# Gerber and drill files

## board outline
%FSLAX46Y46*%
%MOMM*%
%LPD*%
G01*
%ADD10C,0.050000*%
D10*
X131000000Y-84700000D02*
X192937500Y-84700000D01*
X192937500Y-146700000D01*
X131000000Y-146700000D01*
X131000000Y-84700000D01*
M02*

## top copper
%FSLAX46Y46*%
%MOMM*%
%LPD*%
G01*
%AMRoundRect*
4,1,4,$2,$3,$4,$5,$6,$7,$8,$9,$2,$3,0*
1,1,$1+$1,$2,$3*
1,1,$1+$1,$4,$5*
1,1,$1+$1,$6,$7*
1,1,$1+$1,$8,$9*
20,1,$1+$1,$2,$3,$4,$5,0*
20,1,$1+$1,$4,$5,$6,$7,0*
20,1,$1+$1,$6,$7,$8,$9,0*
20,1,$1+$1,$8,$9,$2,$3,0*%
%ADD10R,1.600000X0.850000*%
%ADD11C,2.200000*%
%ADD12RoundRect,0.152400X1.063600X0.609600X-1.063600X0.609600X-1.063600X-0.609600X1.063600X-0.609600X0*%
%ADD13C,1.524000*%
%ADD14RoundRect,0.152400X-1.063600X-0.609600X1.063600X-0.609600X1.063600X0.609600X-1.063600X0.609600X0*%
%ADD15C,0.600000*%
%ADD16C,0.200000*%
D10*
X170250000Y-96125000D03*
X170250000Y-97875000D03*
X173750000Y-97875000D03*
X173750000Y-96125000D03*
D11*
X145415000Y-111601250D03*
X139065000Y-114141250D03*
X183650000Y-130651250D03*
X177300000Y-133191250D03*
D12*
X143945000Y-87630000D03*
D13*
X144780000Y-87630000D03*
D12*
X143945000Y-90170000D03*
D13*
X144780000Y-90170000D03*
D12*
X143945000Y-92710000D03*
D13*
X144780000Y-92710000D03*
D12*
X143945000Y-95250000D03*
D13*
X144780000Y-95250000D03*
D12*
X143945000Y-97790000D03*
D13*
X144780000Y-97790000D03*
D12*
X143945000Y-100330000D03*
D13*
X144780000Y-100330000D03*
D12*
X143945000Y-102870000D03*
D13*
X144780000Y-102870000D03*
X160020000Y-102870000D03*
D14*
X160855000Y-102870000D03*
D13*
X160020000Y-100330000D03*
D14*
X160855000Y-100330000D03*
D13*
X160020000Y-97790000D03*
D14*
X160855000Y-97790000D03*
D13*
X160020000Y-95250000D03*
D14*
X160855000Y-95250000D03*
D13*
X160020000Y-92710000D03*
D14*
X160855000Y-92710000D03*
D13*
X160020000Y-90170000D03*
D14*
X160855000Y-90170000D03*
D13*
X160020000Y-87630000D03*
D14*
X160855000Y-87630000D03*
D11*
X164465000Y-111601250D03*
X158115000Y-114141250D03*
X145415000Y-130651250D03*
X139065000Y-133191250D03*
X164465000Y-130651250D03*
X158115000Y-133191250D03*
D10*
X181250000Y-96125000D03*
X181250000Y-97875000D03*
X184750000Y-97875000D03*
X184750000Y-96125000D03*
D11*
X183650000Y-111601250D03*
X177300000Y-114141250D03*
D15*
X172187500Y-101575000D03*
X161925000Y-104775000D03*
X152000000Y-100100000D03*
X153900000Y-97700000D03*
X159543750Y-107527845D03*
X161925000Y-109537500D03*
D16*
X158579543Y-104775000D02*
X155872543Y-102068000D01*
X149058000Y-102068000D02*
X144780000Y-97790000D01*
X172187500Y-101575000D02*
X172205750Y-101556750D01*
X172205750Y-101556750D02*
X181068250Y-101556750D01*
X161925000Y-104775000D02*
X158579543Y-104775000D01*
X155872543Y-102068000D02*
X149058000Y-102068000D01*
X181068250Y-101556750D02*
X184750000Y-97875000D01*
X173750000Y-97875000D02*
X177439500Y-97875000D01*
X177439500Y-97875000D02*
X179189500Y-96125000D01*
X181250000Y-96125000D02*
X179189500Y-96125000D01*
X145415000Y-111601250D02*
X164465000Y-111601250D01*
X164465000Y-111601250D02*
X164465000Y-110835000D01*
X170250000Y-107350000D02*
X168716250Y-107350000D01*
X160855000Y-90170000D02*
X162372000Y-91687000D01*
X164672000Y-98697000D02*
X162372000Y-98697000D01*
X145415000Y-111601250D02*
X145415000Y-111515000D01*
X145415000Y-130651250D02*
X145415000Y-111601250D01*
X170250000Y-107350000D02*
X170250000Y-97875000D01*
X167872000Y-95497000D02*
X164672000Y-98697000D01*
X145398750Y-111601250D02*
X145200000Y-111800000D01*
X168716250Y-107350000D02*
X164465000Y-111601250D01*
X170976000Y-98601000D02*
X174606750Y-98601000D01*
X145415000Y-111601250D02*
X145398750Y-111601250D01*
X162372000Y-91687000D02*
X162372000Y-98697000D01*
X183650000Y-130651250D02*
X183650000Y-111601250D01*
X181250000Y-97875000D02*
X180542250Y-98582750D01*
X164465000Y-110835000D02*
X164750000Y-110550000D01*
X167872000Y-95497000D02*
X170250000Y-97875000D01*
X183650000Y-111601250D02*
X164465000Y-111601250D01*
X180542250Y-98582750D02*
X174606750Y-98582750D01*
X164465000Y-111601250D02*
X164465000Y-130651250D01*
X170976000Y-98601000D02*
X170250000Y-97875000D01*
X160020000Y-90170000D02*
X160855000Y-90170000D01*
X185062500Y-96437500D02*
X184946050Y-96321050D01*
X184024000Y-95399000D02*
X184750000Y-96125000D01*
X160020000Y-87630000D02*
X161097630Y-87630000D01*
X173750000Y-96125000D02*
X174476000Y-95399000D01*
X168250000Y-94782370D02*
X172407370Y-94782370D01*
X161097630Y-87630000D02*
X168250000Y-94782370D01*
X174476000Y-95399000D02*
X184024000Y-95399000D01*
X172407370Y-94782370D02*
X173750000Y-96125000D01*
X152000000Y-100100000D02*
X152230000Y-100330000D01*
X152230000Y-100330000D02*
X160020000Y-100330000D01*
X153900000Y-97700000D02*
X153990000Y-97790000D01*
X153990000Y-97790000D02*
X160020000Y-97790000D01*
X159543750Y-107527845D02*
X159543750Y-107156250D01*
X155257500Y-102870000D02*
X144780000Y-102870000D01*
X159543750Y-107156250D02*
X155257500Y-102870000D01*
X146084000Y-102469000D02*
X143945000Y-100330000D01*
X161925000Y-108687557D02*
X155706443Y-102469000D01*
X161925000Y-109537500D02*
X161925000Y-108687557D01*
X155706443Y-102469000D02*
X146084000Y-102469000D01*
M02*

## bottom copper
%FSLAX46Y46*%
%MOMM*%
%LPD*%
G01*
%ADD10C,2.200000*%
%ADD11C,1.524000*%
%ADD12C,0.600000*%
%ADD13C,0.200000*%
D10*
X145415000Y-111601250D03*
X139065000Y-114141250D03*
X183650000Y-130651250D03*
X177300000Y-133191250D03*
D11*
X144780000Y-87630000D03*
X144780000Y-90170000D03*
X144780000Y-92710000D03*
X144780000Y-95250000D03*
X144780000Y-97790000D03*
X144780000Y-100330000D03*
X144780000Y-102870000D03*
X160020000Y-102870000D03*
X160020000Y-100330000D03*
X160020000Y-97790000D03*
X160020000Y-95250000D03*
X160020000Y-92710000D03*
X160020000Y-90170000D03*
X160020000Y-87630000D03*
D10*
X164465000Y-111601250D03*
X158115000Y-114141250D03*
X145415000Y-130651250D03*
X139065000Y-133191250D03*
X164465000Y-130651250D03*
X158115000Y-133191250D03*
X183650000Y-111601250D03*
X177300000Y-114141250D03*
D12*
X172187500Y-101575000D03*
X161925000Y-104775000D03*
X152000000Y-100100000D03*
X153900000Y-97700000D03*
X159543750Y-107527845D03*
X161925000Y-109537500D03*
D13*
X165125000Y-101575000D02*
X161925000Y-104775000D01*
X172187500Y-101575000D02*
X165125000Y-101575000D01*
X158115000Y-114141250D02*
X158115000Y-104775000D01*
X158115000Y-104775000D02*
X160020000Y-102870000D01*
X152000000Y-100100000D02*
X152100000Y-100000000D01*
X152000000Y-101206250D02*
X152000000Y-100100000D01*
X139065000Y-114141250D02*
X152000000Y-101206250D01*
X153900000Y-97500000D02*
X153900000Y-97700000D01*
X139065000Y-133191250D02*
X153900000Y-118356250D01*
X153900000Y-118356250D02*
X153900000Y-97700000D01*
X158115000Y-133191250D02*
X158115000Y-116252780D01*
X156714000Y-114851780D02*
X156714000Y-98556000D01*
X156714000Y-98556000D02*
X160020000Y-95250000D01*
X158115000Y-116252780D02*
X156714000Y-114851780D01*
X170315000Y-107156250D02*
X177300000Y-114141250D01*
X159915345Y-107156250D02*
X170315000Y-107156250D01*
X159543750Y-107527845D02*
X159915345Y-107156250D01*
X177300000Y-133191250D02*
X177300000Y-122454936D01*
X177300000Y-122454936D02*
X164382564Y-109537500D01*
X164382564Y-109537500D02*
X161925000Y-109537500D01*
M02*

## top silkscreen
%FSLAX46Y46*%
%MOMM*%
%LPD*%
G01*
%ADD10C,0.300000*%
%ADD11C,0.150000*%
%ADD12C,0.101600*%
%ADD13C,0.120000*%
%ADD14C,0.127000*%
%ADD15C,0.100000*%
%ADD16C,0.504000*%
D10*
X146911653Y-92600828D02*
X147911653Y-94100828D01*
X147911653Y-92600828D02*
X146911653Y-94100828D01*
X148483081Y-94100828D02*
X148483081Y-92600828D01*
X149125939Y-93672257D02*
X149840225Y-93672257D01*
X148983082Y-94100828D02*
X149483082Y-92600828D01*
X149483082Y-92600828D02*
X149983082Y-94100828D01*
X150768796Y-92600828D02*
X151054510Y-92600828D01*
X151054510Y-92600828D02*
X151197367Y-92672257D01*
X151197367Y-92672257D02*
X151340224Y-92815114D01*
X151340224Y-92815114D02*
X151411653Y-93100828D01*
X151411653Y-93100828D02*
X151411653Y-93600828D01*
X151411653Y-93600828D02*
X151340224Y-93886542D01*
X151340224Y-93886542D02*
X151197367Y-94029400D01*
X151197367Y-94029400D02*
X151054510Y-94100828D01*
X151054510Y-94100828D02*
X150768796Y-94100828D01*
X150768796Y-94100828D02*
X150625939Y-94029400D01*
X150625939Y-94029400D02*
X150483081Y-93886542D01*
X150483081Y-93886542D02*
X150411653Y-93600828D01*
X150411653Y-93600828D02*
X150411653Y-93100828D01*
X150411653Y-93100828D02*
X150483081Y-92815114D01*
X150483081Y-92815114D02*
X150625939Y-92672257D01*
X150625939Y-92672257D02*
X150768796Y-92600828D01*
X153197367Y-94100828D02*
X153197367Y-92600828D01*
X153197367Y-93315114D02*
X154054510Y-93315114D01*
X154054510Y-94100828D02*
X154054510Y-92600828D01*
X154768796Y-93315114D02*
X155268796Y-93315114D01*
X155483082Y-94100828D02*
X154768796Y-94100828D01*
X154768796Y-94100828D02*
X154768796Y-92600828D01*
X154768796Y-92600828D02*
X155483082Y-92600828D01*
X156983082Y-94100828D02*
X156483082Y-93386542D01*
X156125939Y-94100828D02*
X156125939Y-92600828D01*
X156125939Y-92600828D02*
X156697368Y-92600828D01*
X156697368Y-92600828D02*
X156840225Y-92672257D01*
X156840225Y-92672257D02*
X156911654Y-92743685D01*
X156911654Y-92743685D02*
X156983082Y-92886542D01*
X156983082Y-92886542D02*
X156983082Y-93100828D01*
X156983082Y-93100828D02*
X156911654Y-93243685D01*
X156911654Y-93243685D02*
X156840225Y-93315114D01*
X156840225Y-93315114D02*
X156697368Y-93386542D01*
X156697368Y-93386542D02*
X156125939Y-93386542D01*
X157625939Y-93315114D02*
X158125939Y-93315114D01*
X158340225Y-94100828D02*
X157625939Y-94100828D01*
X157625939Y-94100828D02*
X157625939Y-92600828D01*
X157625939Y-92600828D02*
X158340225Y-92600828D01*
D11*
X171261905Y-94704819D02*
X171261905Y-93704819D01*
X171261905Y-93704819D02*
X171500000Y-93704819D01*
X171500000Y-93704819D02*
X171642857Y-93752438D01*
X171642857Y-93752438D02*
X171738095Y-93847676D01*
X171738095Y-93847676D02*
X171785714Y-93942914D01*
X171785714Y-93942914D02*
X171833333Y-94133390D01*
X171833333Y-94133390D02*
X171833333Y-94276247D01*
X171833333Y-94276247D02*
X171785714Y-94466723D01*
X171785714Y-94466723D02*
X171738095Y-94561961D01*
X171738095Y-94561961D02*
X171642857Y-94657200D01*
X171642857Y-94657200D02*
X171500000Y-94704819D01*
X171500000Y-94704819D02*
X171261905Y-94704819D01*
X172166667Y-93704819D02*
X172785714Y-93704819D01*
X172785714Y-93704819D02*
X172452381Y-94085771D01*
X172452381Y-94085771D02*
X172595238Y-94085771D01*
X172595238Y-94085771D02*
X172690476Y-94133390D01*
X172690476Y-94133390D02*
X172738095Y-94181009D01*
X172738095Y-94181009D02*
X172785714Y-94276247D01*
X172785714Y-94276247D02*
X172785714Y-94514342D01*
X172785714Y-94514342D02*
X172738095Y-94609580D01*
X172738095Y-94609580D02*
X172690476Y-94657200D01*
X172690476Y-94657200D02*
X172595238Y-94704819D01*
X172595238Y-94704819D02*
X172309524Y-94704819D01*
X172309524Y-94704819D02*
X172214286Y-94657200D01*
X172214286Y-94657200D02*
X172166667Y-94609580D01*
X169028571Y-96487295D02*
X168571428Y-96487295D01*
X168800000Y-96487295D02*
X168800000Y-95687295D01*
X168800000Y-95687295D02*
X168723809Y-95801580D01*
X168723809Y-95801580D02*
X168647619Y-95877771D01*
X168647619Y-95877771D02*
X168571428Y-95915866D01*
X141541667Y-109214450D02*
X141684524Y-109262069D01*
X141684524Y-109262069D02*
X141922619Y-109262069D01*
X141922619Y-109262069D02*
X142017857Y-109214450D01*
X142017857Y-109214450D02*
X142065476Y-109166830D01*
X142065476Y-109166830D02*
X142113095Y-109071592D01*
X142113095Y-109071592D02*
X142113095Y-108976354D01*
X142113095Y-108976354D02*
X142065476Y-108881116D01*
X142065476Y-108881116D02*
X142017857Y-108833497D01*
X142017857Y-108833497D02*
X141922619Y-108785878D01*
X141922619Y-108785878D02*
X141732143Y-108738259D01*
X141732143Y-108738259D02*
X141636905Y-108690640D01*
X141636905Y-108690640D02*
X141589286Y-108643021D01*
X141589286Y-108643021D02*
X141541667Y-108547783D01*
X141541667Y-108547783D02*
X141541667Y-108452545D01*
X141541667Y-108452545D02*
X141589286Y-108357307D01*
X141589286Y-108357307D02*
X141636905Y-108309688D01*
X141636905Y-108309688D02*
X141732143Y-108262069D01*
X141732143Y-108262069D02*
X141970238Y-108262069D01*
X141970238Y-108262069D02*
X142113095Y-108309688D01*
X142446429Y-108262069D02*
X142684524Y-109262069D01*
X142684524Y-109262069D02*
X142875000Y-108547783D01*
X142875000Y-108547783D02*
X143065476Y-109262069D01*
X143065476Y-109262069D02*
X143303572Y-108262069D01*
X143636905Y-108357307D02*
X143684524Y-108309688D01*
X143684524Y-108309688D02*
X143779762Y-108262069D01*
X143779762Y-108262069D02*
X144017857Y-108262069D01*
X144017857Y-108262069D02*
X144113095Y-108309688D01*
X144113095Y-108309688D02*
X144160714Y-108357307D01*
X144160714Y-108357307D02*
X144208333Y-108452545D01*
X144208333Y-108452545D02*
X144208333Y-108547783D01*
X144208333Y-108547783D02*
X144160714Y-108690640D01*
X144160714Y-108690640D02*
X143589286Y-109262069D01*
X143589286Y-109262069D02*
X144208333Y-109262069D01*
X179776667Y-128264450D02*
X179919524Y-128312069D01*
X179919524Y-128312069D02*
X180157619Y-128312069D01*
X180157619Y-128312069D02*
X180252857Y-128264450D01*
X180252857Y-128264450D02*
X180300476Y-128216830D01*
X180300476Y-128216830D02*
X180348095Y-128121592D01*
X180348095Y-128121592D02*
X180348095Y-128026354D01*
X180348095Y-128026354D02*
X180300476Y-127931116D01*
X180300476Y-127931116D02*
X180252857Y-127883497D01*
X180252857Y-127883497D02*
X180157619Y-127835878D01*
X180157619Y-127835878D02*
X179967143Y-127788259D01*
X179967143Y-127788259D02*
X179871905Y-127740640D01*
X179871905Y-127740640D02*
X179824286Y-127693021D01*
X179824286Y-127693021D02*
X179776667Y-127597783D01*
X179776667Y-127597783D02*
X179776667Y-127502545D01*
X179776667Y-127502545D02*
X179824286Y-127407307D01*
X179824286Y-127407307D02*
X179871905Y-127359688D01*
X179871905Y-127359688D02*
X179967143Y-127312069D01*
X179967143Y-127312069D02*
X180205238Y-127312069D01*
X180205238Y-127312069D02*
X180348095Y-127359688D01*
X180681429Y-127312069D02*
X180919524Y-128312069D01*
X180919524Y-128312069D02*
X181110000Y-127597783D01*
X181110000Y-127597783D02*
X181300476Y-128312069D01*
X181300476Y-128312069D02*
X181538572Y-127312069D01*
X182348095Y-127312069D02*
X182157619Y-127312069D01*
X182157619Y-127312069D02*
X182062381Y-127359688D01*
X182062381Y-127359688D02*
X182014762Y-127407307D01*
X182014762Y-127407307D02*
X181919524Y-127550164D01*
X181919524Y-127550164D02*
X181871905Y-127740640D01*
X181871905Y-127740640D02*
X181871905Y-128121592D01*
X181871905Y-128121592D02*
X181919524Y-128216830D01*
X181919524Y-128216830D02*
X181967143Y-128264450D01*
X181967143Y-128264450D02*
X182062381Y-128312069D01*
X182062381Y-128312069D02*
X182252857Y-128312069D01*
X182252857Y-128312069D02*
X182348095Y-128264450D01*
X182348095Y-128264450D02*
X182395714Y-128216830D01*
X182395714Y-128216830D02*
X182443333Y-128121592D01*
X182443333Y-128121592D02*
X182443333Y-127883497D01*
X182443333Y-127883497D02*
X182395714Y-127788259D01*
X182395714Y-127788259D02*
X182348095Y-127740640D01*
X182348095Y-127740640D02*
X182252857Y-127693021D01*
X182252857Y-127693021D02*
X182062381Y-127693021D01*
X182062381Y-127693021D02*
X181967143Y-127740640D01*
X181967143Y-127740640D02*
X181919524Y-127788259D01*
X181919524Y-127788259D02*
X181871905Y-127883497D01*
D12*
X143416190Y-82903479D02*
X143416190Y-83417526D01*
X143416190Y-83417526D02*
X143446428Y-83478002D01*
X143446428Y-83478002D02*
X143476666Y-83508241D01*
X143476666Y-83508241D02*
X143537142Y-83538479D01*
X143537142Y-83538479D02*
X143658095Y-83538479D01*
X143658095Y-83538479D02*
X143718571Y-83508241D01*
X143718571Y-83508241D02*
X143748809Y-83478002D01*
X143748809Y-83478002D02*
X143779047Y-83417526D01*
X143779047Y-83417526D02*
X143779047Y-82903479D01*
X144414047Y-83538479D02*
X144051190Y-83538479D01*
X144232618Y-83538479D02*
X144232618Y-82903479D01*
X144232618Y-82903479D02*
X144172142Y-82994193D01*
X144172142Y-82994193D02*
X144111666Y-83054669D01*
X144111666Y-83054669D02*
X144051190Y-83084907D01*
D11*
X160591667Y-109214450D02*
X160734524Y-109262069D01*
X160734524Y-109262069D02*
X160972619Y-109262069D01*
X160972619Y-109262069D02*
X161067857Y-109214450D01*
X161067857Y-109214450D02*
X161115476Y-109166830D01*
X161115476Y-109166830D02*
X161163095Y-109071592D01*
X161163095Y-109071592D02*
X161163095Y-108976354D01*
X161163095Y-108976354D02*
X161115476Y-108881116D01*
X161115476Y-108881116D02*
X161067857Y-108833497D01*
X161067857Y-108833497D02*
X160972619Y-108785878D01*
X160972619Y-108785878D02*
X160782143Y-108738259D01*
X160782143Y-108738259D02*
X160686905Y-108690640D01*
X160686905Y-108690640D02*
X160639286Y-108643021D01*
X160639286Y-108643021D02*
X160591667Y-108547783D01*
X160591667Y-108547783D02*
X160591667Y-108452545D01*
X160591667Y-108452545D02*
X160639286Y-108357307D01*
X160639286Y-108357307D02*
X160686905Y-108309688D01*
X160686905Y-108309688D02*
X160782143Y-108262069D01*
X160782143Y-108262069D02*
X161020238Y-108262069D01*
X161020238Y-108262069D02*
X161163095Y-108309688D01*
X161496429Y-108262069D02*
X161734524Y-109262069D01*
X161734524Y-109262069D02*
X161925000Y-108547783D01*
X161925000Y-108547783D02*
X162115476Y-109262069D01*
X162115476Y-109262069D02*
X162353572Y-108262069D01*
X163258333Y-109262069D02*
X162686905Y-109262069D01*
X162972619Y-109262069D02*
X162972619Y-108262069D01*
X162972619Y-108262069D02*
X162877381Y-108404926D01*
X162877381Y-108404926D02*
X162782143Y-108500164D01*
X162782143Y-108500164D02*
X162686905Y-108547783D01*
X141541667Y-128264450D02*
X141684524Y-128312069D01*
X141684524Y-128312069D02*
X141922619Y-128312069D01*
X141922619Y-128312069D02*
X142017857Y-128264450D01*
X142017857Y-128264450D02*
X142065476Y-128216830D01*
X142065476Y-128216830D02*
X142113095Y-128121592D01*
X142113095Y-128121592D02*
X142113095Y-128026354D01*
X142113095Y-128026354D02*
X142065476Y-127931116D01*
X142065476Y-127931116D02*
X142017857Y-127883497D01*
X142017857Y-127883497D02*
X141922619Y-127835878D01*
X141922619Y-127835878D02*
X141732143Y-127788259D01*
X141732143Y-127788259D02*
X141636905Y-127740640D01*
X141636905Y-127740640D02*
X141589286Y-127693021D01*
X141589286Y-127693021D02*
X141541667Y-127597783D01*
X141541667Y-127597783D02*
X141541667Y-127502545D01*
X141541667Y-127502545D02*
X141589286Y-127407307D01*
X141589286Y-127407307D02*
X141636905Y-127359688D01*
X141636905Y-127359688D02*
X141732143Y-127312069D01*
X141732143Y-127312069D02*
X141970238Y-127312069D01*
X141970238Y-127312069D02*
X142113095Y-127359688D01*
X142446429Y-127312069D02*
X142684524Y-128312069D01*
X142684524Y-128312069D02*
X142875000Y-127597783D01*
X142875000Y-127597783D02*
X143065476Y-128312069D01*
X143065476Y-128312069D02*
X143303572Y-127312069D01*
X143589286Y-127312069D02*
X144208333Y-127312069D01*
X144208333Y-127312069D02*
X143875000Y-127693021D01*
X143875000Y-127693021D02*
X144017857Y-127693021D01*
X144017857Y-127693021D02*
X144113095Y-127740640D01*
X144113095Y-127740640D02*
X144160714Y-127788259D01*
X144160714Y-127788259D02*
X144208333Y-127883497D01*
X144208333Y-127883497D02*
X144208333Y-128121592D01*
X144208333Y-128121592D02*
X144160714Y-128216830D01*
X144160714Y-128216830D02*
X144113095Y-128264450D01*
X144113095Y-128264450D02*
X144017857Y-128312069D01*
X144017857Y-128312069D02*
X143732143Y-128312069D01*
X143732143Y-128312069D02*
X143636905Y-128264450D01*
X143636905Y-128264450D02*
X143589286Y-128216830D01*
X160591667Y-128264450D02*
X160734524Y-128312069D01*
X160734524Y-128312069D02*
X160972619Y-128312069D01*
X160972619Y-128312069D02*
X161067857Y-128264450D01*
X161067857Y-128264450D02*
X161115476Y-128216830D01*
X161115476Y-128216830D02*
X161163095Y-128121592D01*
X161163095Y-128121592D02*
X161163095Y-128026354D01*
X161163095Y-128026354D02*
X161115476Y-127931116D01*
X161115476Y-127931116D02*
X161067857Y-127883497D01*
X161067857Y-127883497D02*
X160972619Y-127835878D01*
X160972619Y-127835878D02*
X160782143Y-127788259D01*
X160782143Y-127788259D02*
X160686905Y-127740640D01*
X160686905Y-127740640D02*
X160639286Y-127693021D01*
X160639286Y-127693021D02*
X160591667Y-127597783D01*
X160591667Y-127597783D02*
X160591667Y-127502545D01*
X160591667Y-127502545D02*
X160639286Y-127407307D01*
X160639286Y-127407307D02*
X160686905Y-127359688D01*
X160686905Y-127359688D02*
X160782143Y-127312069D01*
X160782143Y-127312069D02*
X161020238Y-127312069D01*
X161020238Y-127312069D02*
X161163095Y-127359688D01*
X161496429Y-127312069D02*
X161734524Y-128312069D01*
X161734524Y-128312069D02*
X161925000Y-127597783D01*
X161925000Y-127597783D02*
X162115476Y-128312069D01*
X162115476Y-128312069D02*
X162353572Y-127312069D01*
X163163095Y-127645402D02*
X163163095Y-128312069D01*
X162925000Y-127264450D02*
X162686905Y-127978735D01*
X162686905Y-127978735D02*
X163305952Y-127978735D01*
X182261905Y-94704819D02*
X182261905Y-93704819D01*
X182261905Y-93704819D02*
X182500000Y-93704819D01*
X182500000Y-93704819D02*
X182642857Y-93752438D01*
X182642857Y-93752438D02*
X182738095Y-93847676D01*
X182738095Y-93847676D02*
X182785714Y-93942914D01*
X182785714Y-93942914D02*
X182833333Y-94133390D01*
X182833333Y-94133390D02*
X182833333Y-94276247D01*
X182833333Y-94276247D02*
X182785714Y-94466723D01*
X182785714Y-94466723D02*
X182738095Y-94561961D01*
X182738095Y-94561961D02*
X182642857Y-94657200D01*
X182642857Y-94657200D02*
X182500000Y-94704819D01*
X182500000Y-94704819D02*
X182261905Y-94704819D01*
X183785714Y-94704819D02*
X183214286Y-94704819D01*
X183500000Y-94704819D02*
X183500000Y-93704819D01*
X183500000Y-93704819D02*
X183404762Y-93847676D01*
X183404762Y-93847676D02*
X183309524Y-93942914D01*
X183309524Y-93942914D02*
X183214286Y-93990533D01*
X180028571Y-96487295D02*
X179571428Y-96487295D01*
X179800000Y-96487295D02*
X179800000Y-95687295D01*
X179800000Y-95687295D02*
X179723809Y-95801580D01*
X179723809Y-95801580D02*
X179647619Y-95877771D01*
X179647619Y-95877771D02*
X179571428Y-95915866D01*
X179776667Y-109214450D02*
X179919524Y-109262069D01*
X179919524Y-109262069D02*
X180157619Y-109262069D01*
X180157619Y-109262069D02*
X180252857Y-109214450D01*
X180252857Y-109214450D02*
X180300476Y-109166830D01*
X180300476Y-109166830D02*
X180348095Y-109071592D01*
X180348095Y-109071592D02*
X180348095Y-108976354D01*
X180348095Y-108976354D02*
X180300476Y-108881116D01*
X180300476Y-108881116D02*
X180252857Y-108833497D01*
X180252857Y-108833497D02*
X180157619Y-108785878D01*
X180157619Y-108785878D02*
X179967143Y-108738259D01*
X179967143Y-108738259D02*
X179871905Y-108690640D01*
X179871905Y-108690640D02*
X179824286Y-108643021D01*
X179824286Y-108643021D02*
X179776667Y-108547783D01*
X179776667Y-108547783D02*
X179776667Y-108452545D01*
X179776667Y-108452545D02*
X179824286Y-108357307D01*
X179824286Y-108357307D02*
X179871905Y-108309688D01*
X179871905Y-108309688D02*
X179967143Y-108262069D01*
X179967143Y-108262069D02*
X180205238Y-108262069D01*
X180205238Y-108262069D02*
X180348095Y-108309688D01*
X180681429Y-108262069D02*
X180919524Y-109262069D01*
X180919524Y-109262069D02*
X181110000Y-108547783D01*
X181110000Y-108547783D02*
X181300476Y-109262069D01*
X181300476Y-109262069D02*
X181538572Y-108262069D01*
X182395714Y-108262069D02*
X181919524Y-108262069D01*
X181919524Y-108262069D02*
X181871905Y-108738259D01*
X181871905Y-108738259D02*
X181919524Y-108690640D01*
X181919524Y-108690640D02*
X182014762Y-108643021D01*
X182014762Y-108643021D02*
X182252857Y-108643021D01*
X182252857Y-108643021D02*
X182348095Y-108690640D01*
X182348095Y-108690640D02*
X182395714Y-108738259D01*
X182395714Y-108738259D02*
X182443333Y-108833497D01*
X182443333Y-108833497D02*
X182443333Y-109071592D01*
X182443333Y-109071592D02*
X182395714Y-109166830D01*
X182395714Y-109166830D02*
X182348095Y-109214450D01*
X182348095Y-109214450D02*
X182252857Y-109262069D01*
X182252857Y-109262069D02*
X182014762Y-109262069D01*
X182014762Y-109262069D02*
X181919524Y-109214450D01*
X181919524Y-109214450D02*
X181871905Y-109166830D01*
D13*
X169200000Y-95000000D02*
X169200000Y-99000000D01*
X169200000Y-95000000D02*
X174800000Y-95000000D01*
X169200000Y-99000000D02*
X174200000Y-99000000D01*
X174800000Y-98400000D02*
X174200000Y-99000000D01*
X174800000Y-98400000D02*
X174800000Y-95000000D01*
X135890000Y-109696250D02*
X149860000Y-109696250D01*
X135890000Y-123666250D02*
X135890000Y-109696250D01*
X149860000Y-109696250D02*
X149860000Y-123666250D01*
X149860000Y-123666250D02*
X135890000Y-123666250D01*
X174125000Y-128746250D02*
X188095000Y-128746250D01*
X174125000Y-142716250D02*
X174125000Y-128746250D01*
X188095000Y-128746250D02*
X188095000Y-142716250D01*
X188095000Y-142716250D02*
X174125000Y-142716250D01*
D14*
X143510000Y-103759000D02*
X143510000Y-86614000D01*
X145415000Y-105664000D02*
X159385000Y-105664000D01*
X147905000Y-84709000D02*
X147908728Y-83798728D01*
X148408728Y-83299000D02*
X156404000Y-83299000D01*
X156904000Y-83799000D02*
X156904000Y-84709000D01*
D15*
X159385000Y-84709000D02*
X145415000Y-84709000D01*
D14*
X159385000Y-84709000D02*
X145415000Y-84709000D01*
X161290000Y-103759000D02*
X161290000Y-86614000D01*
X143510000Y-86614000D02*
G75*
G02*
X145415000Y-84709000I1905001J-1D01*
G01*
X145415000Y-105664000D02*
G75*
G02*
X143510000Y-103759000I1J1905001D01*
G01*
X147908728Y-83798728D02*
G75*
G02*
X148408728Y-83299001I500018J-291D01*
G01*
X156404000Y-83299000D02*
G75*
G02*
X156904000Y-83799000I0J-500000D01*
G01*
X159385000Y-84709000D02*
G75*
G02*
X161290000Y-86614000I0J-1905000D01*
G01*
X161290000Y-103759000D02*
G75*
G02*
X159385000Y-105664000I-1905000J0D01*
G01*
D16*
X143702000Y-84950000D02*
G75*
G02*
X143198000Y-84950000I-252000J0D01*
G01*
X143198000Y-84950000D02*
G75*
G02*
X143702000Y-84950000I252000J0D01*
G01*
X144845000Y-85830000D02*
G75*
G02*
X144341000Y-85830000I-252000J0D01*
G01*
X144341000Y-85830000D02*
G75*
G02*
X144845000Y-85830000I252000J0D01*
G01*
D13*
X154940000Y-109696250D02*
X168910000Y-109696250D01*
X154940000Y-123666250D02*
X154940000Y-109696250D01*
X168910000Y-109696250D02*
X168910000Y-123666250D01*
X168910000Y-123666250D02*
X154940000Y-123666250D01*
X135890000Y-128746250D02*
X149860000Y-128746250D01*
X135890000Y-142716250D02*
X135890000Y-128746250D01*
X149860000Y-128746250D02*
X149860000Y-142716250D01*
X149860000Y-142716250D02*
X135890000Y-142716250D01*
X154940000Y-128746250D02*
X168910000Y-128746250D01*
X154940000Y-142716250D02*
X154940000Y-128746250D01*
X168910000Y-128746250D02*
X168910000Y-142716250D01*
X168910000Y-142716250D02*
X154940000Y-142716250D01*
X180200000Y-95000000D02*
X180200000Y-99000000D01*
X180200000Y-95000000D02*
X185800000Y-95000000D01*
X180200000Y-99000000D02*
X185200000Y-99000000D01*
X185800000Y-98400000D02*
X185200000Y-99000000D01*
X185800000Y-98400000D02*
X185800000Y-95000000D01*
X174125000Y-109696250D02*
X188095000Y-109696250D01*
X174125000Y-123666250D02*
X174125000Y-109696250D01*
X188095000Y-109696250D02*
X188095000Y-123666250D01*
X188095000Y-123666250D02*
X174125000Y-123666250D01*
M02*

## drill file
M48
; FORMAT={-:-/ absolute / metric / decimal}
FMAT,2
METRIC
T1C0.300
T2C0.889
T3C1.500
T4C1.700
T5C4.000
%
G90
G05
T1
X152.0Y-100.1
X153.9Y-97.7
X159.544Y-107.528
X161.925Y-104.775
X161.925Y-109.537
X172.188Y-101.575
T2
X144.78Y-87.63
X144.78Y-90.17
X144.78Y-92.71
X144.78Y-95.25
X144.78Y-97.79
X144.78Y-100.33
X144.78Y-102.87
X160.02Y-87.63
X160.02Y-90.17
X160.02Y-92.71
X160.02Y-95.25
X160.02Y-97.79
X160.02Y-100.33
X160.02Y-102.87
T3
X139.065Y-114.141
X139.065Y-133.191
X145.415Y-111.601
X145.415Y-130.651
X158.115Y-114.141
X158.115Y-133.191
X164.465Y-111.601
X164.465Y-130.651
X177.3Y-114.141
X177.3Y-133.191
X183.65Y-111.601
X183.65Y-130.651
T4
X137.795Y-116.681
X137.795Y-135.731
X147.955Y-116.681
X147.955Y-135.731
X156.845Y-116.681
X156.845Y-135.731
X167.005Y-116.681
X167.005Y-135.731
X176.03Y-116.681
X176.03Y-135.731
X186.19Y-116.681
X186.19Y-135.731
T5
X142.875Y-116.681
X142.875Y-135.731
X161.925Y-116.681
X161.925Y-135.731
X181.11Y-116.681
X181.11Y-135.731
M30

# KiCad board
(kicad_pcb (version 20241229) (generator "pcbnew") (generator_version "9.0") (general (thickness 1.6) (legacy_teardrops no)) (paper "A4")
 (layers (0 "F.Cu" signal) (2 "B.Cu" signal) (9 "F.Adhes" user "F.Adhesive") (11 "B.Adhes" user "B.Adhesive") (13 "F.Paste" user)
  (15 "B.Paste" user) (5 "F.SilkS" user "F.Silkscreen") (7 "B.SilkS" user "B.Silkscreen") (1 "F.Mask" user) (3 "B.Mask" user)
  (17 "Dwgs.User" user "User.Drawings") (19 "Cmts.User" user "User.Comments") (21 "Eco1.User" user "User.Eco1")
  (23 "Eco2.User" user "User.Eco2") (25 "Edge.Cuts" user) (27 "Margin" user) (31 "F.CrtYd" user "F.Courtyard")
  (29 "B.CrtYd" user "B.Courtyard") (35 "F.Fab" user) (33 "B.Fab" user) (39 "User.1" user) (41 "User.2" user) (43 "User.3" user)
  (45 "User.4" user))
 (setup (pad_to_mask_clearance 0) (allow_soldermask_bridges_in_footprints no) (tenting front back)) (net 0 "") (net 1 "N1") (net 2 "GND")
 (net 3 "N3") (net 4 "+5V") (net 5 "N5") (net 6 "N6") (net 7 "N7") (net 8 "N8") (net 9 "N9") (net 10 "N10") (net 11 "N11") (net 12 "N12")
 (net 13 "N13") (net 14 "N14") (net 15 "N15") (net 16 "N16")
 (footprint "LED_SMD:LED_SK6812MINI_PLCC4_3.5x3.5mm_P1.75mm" (layer "F.Cu") (at 172 97)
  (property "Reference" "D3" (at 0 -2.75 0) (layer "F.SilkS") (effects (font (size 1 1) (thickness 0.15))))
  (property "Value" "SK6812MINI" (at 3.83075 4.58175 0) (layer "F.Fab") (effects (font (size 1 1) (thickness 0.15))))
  (fp_line (start -2.8 -2) (end -2.8 2) (stroke (width 0.12) (type default)) (layer "F.SilkS"))
  (fp_line (start -2.8 -2) (end 2.8 -2) (stroke (width 0.12) (type solid)) (layer "F.SilkS"))
  (fp_line (start -2.8 2) (end 2.2 2) (stroke (width 0.12) (type solid)) (layer "F.SilkS"))
  (fp_line (start 2.8 1.4) (end 2.2 2) (stroke (width 0.12) (type default)) (layer "F.SilkS"))
  (fp_line (start 2.8 1.4) (end 2.8 -2) (stroke (width 0.12) (type solid)) (layer "F.SilkS"))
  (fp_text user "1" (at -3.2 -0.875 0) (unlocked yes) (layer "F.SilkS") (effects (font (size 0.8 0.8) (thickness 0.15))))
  (pad "1" smd rect (at -1.75 -0.875) (size 1.6 0.85) (layers "F.Cu" "F.Mask" "F.Paste") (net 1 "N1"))
  (pad "2" smd rect (at -1.75 0.875) (size 1.6 0.85) (layers "F.Cu" "F.Mask" "F.Paste") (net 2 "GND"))
  (pad "3" smd rect (at 1.75 0.875) (size 1.6 0.85) (layers "F.Cu" "F.Mask" "F.Paste") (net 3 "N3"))
  (pad "4" smd rect (at 1.75 -0.875) (size 1.6 0.85) (layers "F.Cu" "F.Mask" "F.Paste") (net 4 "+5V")))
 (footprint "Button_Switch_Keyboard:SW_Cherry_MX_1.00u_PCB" (layer "F.Cu") (at 145.415 111.60125)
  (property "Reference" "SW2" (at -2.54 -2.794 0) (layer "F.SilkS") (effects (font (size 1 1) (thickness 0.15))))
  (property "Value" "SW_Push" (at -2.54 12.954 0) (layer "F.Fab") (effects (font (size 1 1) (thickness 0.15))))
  (fp_line (start -9.525 -1.905) (end 4.445 -1.905) (stroke (width 0.12) (type solid)) (layer "F.SilkS"))
  (fp_line (start -9.525 12.065) (end -9.525 -1.905) (stroke (width 0.12) (type solid)) (layer "F.SilkS"))
  (fp_line (start 4.445 -1.905) (end 4.445 12.065) (stroke (width 0.12) (type solid)) (layer "F.SilkS"))
  (fp_line (start 4.445 12.065) (end -9.525 12.065) (stroke (width 0.12) (type solid)) (layer "F.SilkS"))
  (pad "" np_thru_hole circle (at -7.62 5.08) (size 1.7 1.7) (drill 1.7) (layers "*.Cu" "*.Mask"))
  (pad "" np_thru_hole circle (at -2.54 5.08) (size 4 4) (drill 4) (layers "*.Cu" "*.Mask"))
  (pad "" np_thru_hole circle (at 2.54 5.08) (size 1.7 1.7) (drill 1.7) (layers "*.Cu" "*.Mask"))
  (pad "1" thru_hole circle (at 0 0) (size 2.2 2.2) (drill 1.5) (layers "*.Cu" "*.Mask") (remove_unused_layers no) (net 2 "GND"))
  (pad "2" thru_hole circle (at -6.35 2.54) (size 2.2 2.2) (drill 1.5) (layers "*.Cu" "*.Mask") (remove_unused_layers no) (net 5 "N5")))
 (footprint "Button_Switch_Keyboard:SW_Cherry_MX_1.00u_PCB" (layer "F.Cu") (at 183.65 130.65125)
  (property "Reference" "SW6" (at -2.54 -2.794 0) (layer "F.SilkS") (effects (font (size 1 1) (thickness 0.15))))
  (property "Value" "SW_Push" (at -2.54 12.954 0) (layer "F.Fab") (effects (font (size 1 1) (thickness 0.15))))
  (fp_line (start -9.525 -1.905) (end 4.445 -1.905) (stroke (width 0.12) (type solid)) (layer "F.SilkS"))
  (fp_line (start -9.525 12.065) (end -9.525 -1.905) (stroke (width 0.12) (type solid)) (layer "F.SilkS"))
  (fp_line (start 4.445 -1.905) (end 4.445 12.065) (stroke (width 0.12) (type solid)) (layer "F.SilkS"))
  (fp_line (start 4.445 12.065) (end -9.525 12.065) (stroke (width 0.12) (type solid)) (layer "F.SilkS"))
  (pad "" np_thru_hole circle (at -7.62 5.08) (size 1.7 1.7) (drill 1.7) (layers "*.Cu" "*.Mask"))
  (pad "" np_thru_hole circle (at -2.54 5.08) (size 4 4) (drill 4) (layers "*.Cu" "*.Mask"))
  (pad "" np_thru_hole circle (at 2.54 5.08) (size 1.7 1.7) (drill 1.7) (layers "*.Cu" "*.Mask"))
  (pad "1" thru_hole circle (at 0 0) (size 2.2 2.2) (drill 1.5) (layers "*.Cu" "*.Mask") (remove_unused_layers no) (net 2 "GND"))
  (pad "2" thru_hole circle (at -6.35 2.54) (size 2.2 2.2) (drill 1.5) (layers "*.Cu" "*.Mask") (remove_unused_layers no) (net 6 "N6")))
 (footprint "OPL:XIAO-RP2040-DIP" (layer "F.Cu") (at 152.4 95.25)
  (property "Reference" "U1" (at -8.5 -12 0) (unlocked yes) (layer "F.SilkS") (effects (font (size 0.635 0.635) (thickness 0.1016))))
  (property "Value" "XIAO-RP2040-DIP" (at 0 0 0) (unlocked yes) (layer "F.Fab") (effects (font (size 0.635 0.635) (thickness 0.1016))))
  (fp_line (start -8.89 8.509) (end -8.89 -8.636) (stroke (width 0.127) (type solid)) (layer "F.SilkS"))
  (fp_line (start -6.985 10.414) (end 6.985 10.414) (stroke (width 0.127) (type solid)) (layer "F.SilkS"))
  (fp_line (start -4.495 -10.541) (end -4.491272 -11.451272) (stroke (width 0.127) (type solid)) (layer "F.SilkS"))
  (fp_line (start -3.991272 -11.951) (end 4.004 -11.951) (stroke (width 0.127) (type solid)) (layer "F.SilkS"))
  (fp_line (start 4.504 -11.451) (end 4.504 -10.541) (stroke (width 0.127) (type solid)) (layer "F.SilkS"))
  (fp_line (start 6.985 -10.541) (end -6.985 -10.541) (stroke (width 0.1) (type solid)) (layer "F.SilkS"))
  (fp_line (start 6.985 -10.541) (end -6.985 -10.541) (stroke (width 0.127) (type solid)) (layer "F.SilkS"))
  (fp_line (start 8.89 8.509) (end 8.89 -8.636) (stroke (width 0.127) (type solid)) (layer "F.SilkS"))
  (fp_arc (start -8.89 -8.636) (mid -8.332038 -9.983038) (end -6.985 -10.541) (stroke (width 0.127) (type solid)) (layer "F.SilkS"))
  (fp_arc (start -6.985 10.414) (mid -8.332038 9.856038) (end -8.89 8.509) (stroke (width 0.127) (type solid)) (layer "F.SilkS"))
  (fp_arc (start -4.491272 -11.451272) (mid -4.344728 -11.80464) (end -3.991272 -11.951) (stroke (width 0.127) (type default))
   (layer "F.SilkS"))
  (fp_arc (start 4.004 -11.951) (mid 4.357553 -11.804553) (end 4.504 -11.451) (stroke (width 0.127) (type default)) (layer "F.SilkS"))
  (fp_arc (start 6.985 -10.541) (mid 8.332038 -9.983038) (end 8.89 -8.636) (stroke (width 0.127) (type solid)) (layer "F.SilkS"))
  (fp_arc (start 8.89 8.509) (mid 8.332038 9.856038) (end 6.985 10.414) (stroke (width 0.127) (type solid)) (layer "F.SilkS"))
  (fp_circle (center -8.95 -10.3) (end -8.95 -10.554) (stroke (width 0.5) (type solid)) (fill yes) (layer "F.SilkS"))
  (fp_circle (center -7.807 -9.42) (end -7.807 -9.674) (stroke (width 0.5) (type solid)) (fill yes) (layer "F.SilkS"))
  (pad "1" smd roundrect (at -8.455 -7.62 180) (size 2.432 1.524) (layers "F.Cu" "F.Mask") (roundrect_rratio 0.1) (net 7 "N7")
   (thermal_bridge_angle 45))
  (pad "1" thru_hole circle (at -7.62 -7.62 180) (size 1.524 1.524) (drill 0.889) (layers "*.Cu" "*.Mask") (remove_unused_layers no)
   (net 7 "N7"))
  (pad "2" smd roundrect (at -8.455 -5.08 180) (size 2.432 1.524) (layers "F.Cu" "F.Mask") (roundrect_rratio 0.1) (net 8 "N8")
   (thermal_bridge_angle 45))
  (pad "2" thru_hole circle (at -7.62 -5.08 180) (size 1.524 1.524) (drill 0.889) (layers "*.Cu" "*.Mask") (remove_unused_layers no)
   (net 8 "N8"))
  (pad "3" smd roundrect (at -8.455 -2.54 180) (size 2.432 1.524) (layers "F.Cu" "F.Mask") (roundrect_rratio 0.1) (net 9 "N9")
   (thermal_bridge_angle 45))
  (pad "3" thru_hole circle (at -7.62 -2.54 180) (size 1.524 1.524) (drill 0.889) (layers "*.Cu" "*.Mask") (remove_unused_layers no)
   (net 9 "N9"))
  (pad "4" smd roundrect (at -8.455 0 180) (size 2.432 1.524) (layers "F.Cu" "F.Mask") (roundrect_rratio 0.1) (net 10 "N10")
   (thermal_bridge_angle 45))
  (pad "4" thru_hole circle (at -7.62 0 180) (size 1.524 1.524) (drill 0.889) (layers "*.Cu" "*.Mask") (remove_unused_layers no)
   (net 10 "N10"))
  (pad "5" smd roundrect (at -8.455 2.54 180) (size 2.432 1.524) (layers "F.Cu" "F.Mask") (roundrect_rratio 0.1) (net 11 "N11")
   (thermal_bridge_angle 45))
  (pad "5" thru_hole circle (at -7.62 2.54 180) (size 1.524 1.524) (drill 0.889) (layers "*.Cu" "*.Mask") (remove_unused_layers no)
   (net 11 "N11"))
  (pad "6" smd roundrect (at -8.455 5.08 180) (size 2.432 1.524) (layers "F.Cu" "F.Mask") (roundrect_rratio 0.1) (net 6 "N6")
   (thermal_bridge_angle 45))
  (pad "6" thru_hole circle (at -7.62 5.08 180) (size 1.524 1.524) (drill 0.889) (layers "*.Cu" "*.Mask") (remove_unused_layers no)
   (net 6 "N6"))
  (pad "7" smd roundrect (at -8.455 7.62 180) (size 2.432 1.524) (layers "F.Cu" "F.Mask") (roundrect_rratio 0.1) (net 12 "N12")
   (thermal_bridge_angle 45))
  (pad "7" thru_hole circle (at -7.62 7.62 180) (size 1.524 1.524) (drill 0.889) (layers "*.Cu" "*.Mask") (remove_unused_layers no)
   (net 12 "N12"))
  (pad "8" thru_hole circle (at 7.62 7.62) (size 1.524 1.524) (drill 0.889) (layers "*.Cu" "*.Mask") (remove_unused_layers no)
   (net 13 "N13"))
  (pad "8" smd roundrect (at 8.455 7.62) (size 2.432 1.524) (layers "F.Cu" "F.Mask") (roundrect_rratio 0.1) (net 13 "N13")
   (thermal_bridge_angle 45))
  (pad "9" thru_hole circle (at 7.62 5.08) (size 1.524 1.524) (drill 0.889) (layers "*.Cu" "*.Mask") (remove_unused_layers no) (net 5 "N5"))
  (pad "9" smd roundrect (at 8.455 5.08) (size 2.432 1.524) (layers "F.Cu" "F.Mask") (roundrect_rratio 0.1) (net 5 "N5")
   (thermal_bridge_angle 45))
  (pad "10" thru_hole circle (at 7.62 2.54) (size 1.524 1.524) (drill 0.889) (layers "*.Cu" "*.Mask") (remove_unused_layers no)
   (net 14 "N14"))
  (pad "10" smd roundrect (at 8.455 2.54) (size 2.432 1.524) (layers "F.Cu" "F.Mask") (roundrect_rratio 0.1) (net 14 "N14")
   (thermal_bridge_angle 45))
  (pad "11" thru_hole circle (at 7.62 0) (size 1.524 1.524) (drill 0.889) (layers "*.Cu" "*.Mask") (remove_unused_layers no) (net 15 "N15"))
  (pad "11" smd roundrect (at 8.455 0) (size 2.432 1.524) (layers "F.Cu" "F.Mask") (roundrect_rratio 0.1) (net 15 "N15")
   (thermal_bridge_angle 45))
  (pad "12" thru_hole circle (at 7.62 -2.54) (size 1.524 1.524) (drill 0.889) (layers "*.Cu" "*.Mask") (remove_unused_layers no)
   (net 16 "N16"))
  (pad "12" smd roundrect (at 8.455 -2.54) (size 2.432 1.524) (layers "F.Cu" "F.Mask") (roundrect_rratio 0.1) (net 16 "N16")
   (thermal_bridge_angle 45))
  (pad "13" thru_hole circle (at 7.62 -5.08) (size 1.524 1.524) (drill 0.889) (layers "*.Cu" "*.Mask") (remove_unused_layers no)
   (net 2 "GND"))
  (pad "13" smd roundrect (at 8.455 -5.08) (size 2.432 1.524) (layers "F.Cu" "F.Mask") (roundrect_rratio 0.1) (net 2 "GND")
   (thermal_bridge_angle 45))
  (pad "14" thru_hole circle (at 7.62 -7.62) (size 1.524 1.524) (drill 0.889) (layers "*.Cu" "*.Mask") (remove_unused_layers no)
   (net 4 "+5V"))
  (pad "14" smd roundrect (at 8.455 -7.62) (size 2.432 1.524) (layers "F.Cu" "F.Mask") (roundrect_rratio 0.1) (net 4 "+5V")
   (thermal_bridge_angle 45)))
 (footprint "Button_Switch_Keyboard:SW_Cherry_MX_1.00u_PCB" (layer "F.Cu") (at 164.465 111.60125)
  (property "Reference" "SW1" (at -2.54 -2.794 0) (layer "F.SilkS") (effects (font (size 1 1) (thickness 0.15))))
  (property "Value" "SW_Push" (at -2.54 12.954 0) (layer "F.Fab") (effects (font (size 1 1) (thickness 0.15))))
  (fp_line (start -9.525 -1.905) (end 4.445 -1.905) (stroke (width 0.12) (type solid)) (layer "F.SilkS"))
  (fp_line (start -9.525 12.065) (end -9.525 -1.905) (stroke (width 0.12) (type solid)) (layer "F.SilkS"))
  (fp_line (start 4.445 -1.905) (end 4.445 12.065) (stroke (width 0.12) (type solid)) (layer "F.SilkS"))
  (fp_line (start 4.445 12.065) (end -9.525 12.065) (stroke (width 0.12) (type solid)) (layer "F.SilkS"))
  (pad "" np_thru_hole circle (at -7.62 5.08) (size 1.7 1.7) (drill 1.7) (layers "*.Cu" "*.Mask"))
  (pad "" np_thru_hole circle (at -2.54 5.08) (size 4 4) (drill 4) (layers "*.Cu" "*.Mask"))
  (pad "" np_thru_hole circle (at 2.54 5.08) (size 1.7 1.7) (drill 1.7) (layers "*.Cu" "*.Mask"))
  (pad "1" thru_hole circle (at 0 0) (size 2.2 2.2) (drill 1.5) (layers "*.Cu" "*.Mask") (remove_unused_layers no) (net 2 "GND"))
  (pad "2" thru_hole circle (at -6.35 2.54) (size 2.2 2.2) (drill 1.5) (layers "*.Cu" "*.Mask") (remove_unused_layers no) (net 13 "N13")))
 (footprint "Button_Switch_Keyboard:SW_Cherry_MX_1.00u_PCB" (layer "F.Cu") (at 145.415 130.65125)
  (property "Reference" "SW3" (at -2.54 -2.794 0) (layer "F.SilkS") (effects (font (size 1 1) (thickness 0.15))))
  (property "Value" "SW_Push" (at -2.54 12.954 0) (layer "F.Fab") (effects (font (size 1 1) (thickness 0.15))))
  (fp_line (start -9.525 -1.905) (end 4.445 -1.905) (stroke (width 0.12) (type solid)) (layer "F.SilkS"))
  (fp_line (start -9.525 12.065) (end -9.525 -1.905) (stroke (width 0.12) (type solid)) (layer "F.SilkS"))
  (fp_line (start 4.445 -1.905) (end 4.445 12.065) (stroke (width 0.12) (type solid)) (layer "F.SilkS"))
  (fp_line (start 4.445 12.065) (end -9.525 12.065) (stroke (width 0.12) (type solid)) (layer "F.SilkS"))
  (pad "" np_thru_hole circle (at -7.62 5.08) (size 1.7 1.7) (drill 1.7) (layers "*.Cu" "*.Mask"))
  (pad "" np_thru_hole circle (at -2.54 5.08) (size 4 4) (drill 4) (layers "*.Cu" "*.Mask"))
  (pad "" np_thru_hole circle (at 2.54 5.08) (size 1.7 1.7) (drill 1.7) (layers "*.Cu" "*.Mask"))
  (pad "1" thru_hole circle (at 0 0) (size 2.2 2.2) (drill 1.5) (layers "*.Cu" "*.Mask") (remove_unused_layers no) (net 2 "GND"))
  (pad "2" thru_hole circle (at -6.35 2.54) (size 2.2 2.2) (drill 1.5) (layers "*.Cu" "*.Mask") (remove_unused_layers no) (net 14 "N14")))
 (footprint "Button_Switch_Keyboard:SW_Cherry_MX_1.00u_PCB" (layer "F.Cu") (at 164.465 130.65125)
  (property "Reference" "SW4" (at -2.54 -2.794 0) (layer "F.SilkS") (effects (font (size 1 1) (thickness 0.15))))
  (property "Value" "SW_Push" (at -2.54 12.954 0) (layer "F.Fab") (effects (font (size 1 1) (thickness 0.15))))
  (fp_line (start -9.525 -1.905) (end 4.445 -1.905) (stroke (width 0.12) (type solid)) (layer "F.SilkS"))
  (fp_line (start -9.525 12.065) (end -9.525 -1.905) (stroke (width 0.12) (type solid)) (layer "F.SilkS"))
  (fp_line (start 4.445 -1.905) (end 4.445 12.065) (stroke (width 0.12) (type solid)) (layer "F.SilkS"))
  (fp_line (start 4.445 12.065) (end -9.525 12.065) (stroke (width 0.12) (type solid)) (layer "F.SilkS"))
  (pad "" np_thru_hole circle (at -7.62 5.08) (size 1.7 1.7) (drill 1.7) (layers "*.Cu" "*.Mask"))
  (pad "" np_thru_hole circle (at -2.54 5.08) (size 4 4) (drill 4) (layers "*.Cu" "*.Mask"))
  (pad "" np_thru_hole circle (at 2.54 5.08) (size 1.7 1.7) (drill 1.7) (layers "*.Cu" "*.Mask"))
  (pad "1" thru_hole circle (at 0 0) (size 2.2 2.2) (drill 1.5) (layers "*.Cu" "*.Mask") (remove_unused_layers no) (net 2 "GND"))
  (pad "2" thru_hole circle (at -6.35 2.54) (size 2.2 2.2) (drill 1.5) (layers "*.Cu" "*.Mask") (remove_unused_layers no) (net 15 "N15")))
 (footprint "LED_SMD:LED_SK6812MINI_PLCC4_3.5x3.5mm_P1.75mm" (layer "F.Cu") (at 183 97)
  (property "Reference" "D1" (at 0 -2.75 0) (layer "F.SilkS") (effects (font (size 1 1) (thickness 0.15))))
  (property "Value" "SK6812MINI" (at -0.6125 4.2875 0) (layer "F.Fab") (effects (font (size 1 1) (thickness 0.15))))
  (fp_line (start -2.8 -2) (end -2.8 2) (stroke (width 0.12) (type default)) (layer "F.SilkS"))
  (fp_line (start -2.8 -2) (end 2.8 -2) (stroke (width 0.12) (type solid)) (layer "F.SilkS"))
  (fp_line (start -2.8 2) (end 2.2 2) (stroke (width 0.12) (type solid)) (layer "F.SilkS"))
  (fp_line (start 2.8 1.4) (end 2.2 2) (stroke (width 0.12) (type default)) (layer "F.SilkS"))
  (fp_line (start 2.8 1.4) (end 2.8 -2) (stroke (width 0.12) (type solid)) (layer "F.SilkS"))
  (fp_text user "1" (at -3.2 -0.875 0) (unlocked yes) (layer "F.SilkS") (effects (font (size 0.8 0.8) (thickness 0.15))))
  (pad "1" smd rect (at -1.75 -0.875) (size 1.6 0.85) (layers "F.Cu" "F.Mask" "F.Paste") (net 3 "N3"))
  (pad "2" smd rect (at -1.75 0.875) (size 1.6 0.85) (layers "F.Cu" "F.Mask" "F.Paste") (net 2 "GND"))
  (pad "3" smd rect (at 1.75 0.875) (size 1.6 0.85) (layers "F.Cu" "F.Mask" "F.Paste") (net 11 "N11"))
  (pad "4" smd rect (at 1.75 -0.875) (size 1.6 0.85) (layers "F.Cu" "F.Mask" "F.Paste") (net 4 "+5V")))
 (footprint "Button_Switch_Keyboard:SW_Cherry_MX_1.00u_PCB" (layer "F.Cu") (at 183.65 111.60125)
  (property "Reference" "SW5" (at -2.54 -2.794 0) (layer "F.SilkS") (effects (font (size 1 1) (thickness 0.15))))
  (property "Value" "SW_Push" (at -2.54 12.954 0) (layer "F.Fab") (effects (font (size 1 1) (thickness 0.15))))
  (fp_line (start -9.525 -1.905) (end 4.445 -1.905) (stroke (width 0.12) (type solid)) (layer "F.SilkS"))
  (fp_line (start -9.525 12.065) (end -9.525 -1.905) (stroke (width 0.12) (type solid)) (layer "F.SilkS"))
  (fp_line (start 4.445 -1.905) (end 4.445 12.065) (stroke (width 0.12) (type solid)) (layer "F.SilkS"))
  (fp_line (start 4.445 12.065) (end -9.525 12.065) (stroke (width 0.12) (type solid)) (layer "F.SilkS"))
  (pad "" np_thru_hole circle (at -7.62 5.08) (size 1.7 1.7) (drill 1.7) (layers "*.Cu" "*.Mask"))
  (pad "" np_thru_hole circle (at -2.54 5.08) (size 4 4) (drill 4) (layers "*.Cu" "*.Mask"))
  (pad "" np_thru_hole circle (at 2.54 5.08) (size 1.7 1.7) (drill 1.7) (layers "*.Cu" "*.Mask"))
  (pad "1" thru_hole circle (at 0 0) (size 2.2 2.2) (drill 1.5) (layers "*.Cu" "*.Mask") (remove_unused_layers no) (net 2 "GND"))
  (pad "2" thru_hole circle (at -6.35 2.54) (size 2.2 2.2) (drill 1.5) (layers "*.Cu" "*.Mask") (remove_unused_layers no) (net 12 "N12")))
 (gr_rect (start 131 84.7) (end 192.9375 146.7) (stroke (width 0.05) (type default)) (fill no) (layer "Edge.Cuts"))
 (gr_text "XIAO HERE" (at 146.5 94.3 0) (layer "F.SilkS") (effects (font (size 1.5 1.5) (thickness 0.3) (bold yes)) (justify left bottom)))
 (segment (start 158.579543 104.775) (end 155.872543 102.068) (width 0.2) (layer "F.Cu") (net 11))
 (segment (start 149.058 102.068) (end 144.78 97.79) (width 0.2) (layer "F.Cu") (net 11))
 (segment (start 172.1875 101.575) (end 172.20575 101.55675) (width 0.2) (layer "F.Cu") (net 11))
 (segment (start 172.20575 101.55675) (end 181.06825 101.55675) (width 0.2) (layer "F.Cu") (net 11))
 (segment (start 161.925 104.775) (end 158.579543 104.775) (width 0.2) (layer "F.Cu") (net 11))
 (segment (start 155.872543 102.068) (end 149.058 102.068) (width 0.2) (layer "F.Cu") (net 11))
 (segment (start 181.06825 101.55675) (end 184.75 97.875) (width 0.2) (layer "F.Cu") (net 11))
 (via (at 172.1875 101.575) (size 0.6) (drill 0.3) (layers "F.Cu" "B.Cu") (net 11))
 (via (at 161.925 104.775) (size 0.6) (drill 0.3) (layers "F.Cu" "B.Cu") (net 11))
 (segment (start 165.125 101.575) (end 161.925 104.775) (width 0.2) (layer "B.Cu") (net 11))
 (segment (start 172.1875 101.575) (end 165.125 101.575) (width 0.2) (layer "B.Cu") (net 11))
 (segment (start 173.75 97.875) (end 177.4395 97.875) (width 0.2) (layer "F.Cu") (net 3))
 (segment (start 177.4395 97.875) (end 179.1895 96.125) (width 0.2) (layer "F.Cu") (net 3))
 (segment (start 181.25 96.125) (end 179.1895 96.125) (width 0.2) (layer "F.Cu") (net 3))
 (segment (start 145.415 111.60125) (end 164.465 111.60125) (width 0.2) (layer "F.Cu") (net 2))
 (segment (start 164.465 111.60125) (end 164.465 110.835) (width 0.2) (layer "F.Cu") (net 2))
 (segment (start 170.25 107.35) (end 168.71625 107.35) (width 0.2) (layer "F.Cu") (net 2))
 (segment (start 160.855 90.17) (end 162.372 91.687) (width 0.2) (layer "F.Cu") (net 2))
 (segment (start 164.672 98.697) (end 162.372 98.697) (width 0.2) (layer "F.Cu") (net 2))
 (segment (start 145.415 111.60125) (end 145.415 111.515) (width 0.2) (layer "F.Cu") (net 2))
 (segment (start 145.415 130.65125) (end 145.415 111.60125) (width 0.2) (layer "F.Cu") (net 2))
 (segment (start 170.25 107.35) (end 170.25 97.875) (width 0.2) (layer "F.Cu") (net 2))
 (segment (start 167.872 95.497) (end 164.672 98.697) (width 0.2) (layer "F.Cu") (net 2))
 (segment (start 145.39875 111.60125) (end 145.2 111.8) (width 0.2) (layer "F.Cu") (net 2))
 (segment (start 168.71625 107.35) (end 164.465 111.60125) (width 0.2) (layer "F.Cu") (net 2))
 (segment (start 170.976 98.601) (end 174.60675 98.601) (width 0.2) (layer "F.Cu") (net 2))
 (segment (start 145.415 111.60125) (end 145.39875 111.60125) (width 0.2) (layer "F.Cu") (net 2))
 (segment (start 162.372 91.687) (end 162.372 98.697) (width 0.2) (layer "F.Cu") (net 2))
 (segment (start 183.65 130.65125) (end 183.65 111.60125) (width 0.2) (layer "F.Cu") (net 2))
 (segment (start 181.25 97.875) (end 180.54225 98.58275) (width 0.2) (layer "F.Cu") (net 2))
 (segment (start 164.465 110.835) (end 164.75 110.55) (width 0.2) (layer "F.Cu") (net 2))
 (segment (start 167.872 95.497) (end 170.25 97.875) (width 0.2) (layer "F.Cu") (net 2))
 (segment (start 183.65 111.60125) (end 164.465 111.60125) (width 0.2) (layer "F.Cu") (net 2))
 (segment (start 180.54225 98.58275) (end 174.60675 98.58275) (width 0.2) (layer "F.Cu") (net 2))
 (segment (start 164.465 111.60125) (end 164.465 130.65125) (width 0.2) (layer "F.Cu") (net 2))
 (segment (start 170.976 98.601) (end 170.25 97.875) (width 0.2) (layer "F.Cu") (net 2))
 (segment (start 160.02 90.17) (end 160.855 90.17) (width 0.2) (layer "F.Cu") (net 2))
 (segment (start 185.0625 96.4375) (end 184.94605 96.32105) (width 0.2) (layer "F.Cu") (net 4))
 (segment (start 184.024 95.399) (end 184.75 96.125) (width 0.2) (layer "F.Cu") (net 4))
 (segment (start 160.02 87.63) (end 161.09763 87.63) (width 0.2) (layer "F.Cu") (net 4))
 (segment (start 173.75 96.125) (end 174.476 95.399) (width 0.2) (layer "F.Cu") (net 4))
 (segment (start 168.25 94.78237) (end 172.40737 94.78237) (width 0.2) (layer "F.Cu") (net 4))
 (segment (start 161.09763 87.63) (end 168.25 94.78237) (width 0.2) (layer "F.Cu") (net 4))
 (segment (start 174.476 95.399) (end 184.024 95.399) (width 0.2) (layer "F.Cu") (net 4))
 (segment (start 172.40737 94.78237) (end 173.75 96.125) (width 0.2) (layer "F.Cu") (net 4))
 (segment (start 158.115 114.14125) (end 158.115 104.775) (width 0.2) (layer "B.Cu") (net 13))
 (segment (start 158.115 104.775) (end 160.02 102.87) (width 0.2) (layer "B.Cu") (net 13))
 (segment (start 152 100.1) (end 152.23 100.33) (width 0.2) (layer "F.Cu") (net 5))
 (segment (start 152.23 100.33) (end 160.02 100.33) (width 0.2) (layer "F.Cu") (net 5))
 (via (at 152 100.1) (size 0.6) (drill 0.3) (layers "F.Cu" "B.Cu") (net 5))
 (segment (start 152 100.1) (end 152.1 100) (width 0.2) (layer "B.Cu") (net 5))
 (segment (start 152 101.20625) (end 152 100.1) (width 0.2) (layer "B.Cu") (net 5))
 (segment (start 139.065 114.14125) (end 152 101.20625) (width 0.2) (layer "B.Cu") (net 5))
 (segment (start 153.9 97.7) (end 153.99 97.79) (width 0.2) (layer "F.Cu") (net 14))
 (segment (start 153.99 97.79) (end 160.02 97.79) (width 0.2) (layer "F.Cu") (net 14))
 (via (at 153.9 97.7) (size 0.6) (drill 0.3) (layers "F.Cu" "B.Cu") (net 14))
 (segment (start 153.9 97.5) (end 153.9 97.7) (width 0.2) (layer "B.Cu") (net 14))
 (segment (start 139.065 133.19125) (end 153.9 118.35625) (width 0.2) (layer "B.Cu") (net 14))
 (segment (start 153.9 118.35625) (end 153.9 97.7) (width 0.2) (layer "B.Cu") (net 14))
 (segment (start 158.115 133.19125) (end 158.115 116.25278) (width 0.2) (layer "B.Cu") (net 15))
 (segment (start 156.714 114.85178) (end 156.714 98.556) (width 0.2) (layer "B.Cu") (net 15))
 (segment (start 156.714 98.556) (end 160.02 95.25) (width 0.2) (layer "B.Cu") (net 15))
 (segment (start 158.115 116.25278) (end 156.714 114.85178) (width 0.2) (layer "B.Cu") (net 15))
 (segment (start 159.54375 107.527845) (end 159.54375 107.15625) (width 0.2) (layer "F.Cu") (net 12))
 (segment (start 155.2575 102.87) (end 144.78 102.87) (width 0.2) (layer "F.Cu") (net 12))
 (segment (start 159.54375 107.15625) (end 155.2575 102.87) (width 0.2) (layer "F.Cu") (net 12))
 (via (at 159.54375 107.527845) (size 0.6) (drill 0.3) (layers "F.Cu" "B.Cu") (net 12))
 (segment (start 170.315 107.15625) (end 177.3 114.14125) (width 0.2) (layer "B.Cu") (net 12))
 (segment (start 159.915345 107.15625) (end 170.315 107.15625) (width 0.2) (layer "B.Cu") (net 12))
 (segment (start 159.54375 107.527845) (end 159.915345 107.15625) (width 0.2) (layer "B.Cu") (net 12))
 (segment (start 146.084 102.469) (end 143.945 100.33) (width 0.2) (layer "F.Cu") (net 6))
 (segment (start 161.925 108.687557) (end 155.706443 102.469) (width 0.2) (layer "F.Cu") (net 6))
 (segment (start 161.925 109.5375) (end 161.925 108.687557) (width 0.2) (layer "F.Cu") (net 6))
 (segment (start 155.706443 102.469) (end 146.084 102.469) (width 0.2) (layer "F.Cu") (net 6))
 (via (at 161.925 109.5375) (size 0.6) (drill 0.3) (layers "F.Cu" "B.Cu") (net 6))
 (segment (start 177.3 133.19125) (end 177.3 122.454936) (width 0.2) (layer "B.Cu") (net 6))
 (segment (start 177.3 122.454936) (end 164.382564 109.5375) (width 0.2) (layer "B.Cu") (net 6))
 (segment (start 164.382564 109.5375) (end 161.925 109.5375) (width 0.2) (layer "B.Cu") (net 6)))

